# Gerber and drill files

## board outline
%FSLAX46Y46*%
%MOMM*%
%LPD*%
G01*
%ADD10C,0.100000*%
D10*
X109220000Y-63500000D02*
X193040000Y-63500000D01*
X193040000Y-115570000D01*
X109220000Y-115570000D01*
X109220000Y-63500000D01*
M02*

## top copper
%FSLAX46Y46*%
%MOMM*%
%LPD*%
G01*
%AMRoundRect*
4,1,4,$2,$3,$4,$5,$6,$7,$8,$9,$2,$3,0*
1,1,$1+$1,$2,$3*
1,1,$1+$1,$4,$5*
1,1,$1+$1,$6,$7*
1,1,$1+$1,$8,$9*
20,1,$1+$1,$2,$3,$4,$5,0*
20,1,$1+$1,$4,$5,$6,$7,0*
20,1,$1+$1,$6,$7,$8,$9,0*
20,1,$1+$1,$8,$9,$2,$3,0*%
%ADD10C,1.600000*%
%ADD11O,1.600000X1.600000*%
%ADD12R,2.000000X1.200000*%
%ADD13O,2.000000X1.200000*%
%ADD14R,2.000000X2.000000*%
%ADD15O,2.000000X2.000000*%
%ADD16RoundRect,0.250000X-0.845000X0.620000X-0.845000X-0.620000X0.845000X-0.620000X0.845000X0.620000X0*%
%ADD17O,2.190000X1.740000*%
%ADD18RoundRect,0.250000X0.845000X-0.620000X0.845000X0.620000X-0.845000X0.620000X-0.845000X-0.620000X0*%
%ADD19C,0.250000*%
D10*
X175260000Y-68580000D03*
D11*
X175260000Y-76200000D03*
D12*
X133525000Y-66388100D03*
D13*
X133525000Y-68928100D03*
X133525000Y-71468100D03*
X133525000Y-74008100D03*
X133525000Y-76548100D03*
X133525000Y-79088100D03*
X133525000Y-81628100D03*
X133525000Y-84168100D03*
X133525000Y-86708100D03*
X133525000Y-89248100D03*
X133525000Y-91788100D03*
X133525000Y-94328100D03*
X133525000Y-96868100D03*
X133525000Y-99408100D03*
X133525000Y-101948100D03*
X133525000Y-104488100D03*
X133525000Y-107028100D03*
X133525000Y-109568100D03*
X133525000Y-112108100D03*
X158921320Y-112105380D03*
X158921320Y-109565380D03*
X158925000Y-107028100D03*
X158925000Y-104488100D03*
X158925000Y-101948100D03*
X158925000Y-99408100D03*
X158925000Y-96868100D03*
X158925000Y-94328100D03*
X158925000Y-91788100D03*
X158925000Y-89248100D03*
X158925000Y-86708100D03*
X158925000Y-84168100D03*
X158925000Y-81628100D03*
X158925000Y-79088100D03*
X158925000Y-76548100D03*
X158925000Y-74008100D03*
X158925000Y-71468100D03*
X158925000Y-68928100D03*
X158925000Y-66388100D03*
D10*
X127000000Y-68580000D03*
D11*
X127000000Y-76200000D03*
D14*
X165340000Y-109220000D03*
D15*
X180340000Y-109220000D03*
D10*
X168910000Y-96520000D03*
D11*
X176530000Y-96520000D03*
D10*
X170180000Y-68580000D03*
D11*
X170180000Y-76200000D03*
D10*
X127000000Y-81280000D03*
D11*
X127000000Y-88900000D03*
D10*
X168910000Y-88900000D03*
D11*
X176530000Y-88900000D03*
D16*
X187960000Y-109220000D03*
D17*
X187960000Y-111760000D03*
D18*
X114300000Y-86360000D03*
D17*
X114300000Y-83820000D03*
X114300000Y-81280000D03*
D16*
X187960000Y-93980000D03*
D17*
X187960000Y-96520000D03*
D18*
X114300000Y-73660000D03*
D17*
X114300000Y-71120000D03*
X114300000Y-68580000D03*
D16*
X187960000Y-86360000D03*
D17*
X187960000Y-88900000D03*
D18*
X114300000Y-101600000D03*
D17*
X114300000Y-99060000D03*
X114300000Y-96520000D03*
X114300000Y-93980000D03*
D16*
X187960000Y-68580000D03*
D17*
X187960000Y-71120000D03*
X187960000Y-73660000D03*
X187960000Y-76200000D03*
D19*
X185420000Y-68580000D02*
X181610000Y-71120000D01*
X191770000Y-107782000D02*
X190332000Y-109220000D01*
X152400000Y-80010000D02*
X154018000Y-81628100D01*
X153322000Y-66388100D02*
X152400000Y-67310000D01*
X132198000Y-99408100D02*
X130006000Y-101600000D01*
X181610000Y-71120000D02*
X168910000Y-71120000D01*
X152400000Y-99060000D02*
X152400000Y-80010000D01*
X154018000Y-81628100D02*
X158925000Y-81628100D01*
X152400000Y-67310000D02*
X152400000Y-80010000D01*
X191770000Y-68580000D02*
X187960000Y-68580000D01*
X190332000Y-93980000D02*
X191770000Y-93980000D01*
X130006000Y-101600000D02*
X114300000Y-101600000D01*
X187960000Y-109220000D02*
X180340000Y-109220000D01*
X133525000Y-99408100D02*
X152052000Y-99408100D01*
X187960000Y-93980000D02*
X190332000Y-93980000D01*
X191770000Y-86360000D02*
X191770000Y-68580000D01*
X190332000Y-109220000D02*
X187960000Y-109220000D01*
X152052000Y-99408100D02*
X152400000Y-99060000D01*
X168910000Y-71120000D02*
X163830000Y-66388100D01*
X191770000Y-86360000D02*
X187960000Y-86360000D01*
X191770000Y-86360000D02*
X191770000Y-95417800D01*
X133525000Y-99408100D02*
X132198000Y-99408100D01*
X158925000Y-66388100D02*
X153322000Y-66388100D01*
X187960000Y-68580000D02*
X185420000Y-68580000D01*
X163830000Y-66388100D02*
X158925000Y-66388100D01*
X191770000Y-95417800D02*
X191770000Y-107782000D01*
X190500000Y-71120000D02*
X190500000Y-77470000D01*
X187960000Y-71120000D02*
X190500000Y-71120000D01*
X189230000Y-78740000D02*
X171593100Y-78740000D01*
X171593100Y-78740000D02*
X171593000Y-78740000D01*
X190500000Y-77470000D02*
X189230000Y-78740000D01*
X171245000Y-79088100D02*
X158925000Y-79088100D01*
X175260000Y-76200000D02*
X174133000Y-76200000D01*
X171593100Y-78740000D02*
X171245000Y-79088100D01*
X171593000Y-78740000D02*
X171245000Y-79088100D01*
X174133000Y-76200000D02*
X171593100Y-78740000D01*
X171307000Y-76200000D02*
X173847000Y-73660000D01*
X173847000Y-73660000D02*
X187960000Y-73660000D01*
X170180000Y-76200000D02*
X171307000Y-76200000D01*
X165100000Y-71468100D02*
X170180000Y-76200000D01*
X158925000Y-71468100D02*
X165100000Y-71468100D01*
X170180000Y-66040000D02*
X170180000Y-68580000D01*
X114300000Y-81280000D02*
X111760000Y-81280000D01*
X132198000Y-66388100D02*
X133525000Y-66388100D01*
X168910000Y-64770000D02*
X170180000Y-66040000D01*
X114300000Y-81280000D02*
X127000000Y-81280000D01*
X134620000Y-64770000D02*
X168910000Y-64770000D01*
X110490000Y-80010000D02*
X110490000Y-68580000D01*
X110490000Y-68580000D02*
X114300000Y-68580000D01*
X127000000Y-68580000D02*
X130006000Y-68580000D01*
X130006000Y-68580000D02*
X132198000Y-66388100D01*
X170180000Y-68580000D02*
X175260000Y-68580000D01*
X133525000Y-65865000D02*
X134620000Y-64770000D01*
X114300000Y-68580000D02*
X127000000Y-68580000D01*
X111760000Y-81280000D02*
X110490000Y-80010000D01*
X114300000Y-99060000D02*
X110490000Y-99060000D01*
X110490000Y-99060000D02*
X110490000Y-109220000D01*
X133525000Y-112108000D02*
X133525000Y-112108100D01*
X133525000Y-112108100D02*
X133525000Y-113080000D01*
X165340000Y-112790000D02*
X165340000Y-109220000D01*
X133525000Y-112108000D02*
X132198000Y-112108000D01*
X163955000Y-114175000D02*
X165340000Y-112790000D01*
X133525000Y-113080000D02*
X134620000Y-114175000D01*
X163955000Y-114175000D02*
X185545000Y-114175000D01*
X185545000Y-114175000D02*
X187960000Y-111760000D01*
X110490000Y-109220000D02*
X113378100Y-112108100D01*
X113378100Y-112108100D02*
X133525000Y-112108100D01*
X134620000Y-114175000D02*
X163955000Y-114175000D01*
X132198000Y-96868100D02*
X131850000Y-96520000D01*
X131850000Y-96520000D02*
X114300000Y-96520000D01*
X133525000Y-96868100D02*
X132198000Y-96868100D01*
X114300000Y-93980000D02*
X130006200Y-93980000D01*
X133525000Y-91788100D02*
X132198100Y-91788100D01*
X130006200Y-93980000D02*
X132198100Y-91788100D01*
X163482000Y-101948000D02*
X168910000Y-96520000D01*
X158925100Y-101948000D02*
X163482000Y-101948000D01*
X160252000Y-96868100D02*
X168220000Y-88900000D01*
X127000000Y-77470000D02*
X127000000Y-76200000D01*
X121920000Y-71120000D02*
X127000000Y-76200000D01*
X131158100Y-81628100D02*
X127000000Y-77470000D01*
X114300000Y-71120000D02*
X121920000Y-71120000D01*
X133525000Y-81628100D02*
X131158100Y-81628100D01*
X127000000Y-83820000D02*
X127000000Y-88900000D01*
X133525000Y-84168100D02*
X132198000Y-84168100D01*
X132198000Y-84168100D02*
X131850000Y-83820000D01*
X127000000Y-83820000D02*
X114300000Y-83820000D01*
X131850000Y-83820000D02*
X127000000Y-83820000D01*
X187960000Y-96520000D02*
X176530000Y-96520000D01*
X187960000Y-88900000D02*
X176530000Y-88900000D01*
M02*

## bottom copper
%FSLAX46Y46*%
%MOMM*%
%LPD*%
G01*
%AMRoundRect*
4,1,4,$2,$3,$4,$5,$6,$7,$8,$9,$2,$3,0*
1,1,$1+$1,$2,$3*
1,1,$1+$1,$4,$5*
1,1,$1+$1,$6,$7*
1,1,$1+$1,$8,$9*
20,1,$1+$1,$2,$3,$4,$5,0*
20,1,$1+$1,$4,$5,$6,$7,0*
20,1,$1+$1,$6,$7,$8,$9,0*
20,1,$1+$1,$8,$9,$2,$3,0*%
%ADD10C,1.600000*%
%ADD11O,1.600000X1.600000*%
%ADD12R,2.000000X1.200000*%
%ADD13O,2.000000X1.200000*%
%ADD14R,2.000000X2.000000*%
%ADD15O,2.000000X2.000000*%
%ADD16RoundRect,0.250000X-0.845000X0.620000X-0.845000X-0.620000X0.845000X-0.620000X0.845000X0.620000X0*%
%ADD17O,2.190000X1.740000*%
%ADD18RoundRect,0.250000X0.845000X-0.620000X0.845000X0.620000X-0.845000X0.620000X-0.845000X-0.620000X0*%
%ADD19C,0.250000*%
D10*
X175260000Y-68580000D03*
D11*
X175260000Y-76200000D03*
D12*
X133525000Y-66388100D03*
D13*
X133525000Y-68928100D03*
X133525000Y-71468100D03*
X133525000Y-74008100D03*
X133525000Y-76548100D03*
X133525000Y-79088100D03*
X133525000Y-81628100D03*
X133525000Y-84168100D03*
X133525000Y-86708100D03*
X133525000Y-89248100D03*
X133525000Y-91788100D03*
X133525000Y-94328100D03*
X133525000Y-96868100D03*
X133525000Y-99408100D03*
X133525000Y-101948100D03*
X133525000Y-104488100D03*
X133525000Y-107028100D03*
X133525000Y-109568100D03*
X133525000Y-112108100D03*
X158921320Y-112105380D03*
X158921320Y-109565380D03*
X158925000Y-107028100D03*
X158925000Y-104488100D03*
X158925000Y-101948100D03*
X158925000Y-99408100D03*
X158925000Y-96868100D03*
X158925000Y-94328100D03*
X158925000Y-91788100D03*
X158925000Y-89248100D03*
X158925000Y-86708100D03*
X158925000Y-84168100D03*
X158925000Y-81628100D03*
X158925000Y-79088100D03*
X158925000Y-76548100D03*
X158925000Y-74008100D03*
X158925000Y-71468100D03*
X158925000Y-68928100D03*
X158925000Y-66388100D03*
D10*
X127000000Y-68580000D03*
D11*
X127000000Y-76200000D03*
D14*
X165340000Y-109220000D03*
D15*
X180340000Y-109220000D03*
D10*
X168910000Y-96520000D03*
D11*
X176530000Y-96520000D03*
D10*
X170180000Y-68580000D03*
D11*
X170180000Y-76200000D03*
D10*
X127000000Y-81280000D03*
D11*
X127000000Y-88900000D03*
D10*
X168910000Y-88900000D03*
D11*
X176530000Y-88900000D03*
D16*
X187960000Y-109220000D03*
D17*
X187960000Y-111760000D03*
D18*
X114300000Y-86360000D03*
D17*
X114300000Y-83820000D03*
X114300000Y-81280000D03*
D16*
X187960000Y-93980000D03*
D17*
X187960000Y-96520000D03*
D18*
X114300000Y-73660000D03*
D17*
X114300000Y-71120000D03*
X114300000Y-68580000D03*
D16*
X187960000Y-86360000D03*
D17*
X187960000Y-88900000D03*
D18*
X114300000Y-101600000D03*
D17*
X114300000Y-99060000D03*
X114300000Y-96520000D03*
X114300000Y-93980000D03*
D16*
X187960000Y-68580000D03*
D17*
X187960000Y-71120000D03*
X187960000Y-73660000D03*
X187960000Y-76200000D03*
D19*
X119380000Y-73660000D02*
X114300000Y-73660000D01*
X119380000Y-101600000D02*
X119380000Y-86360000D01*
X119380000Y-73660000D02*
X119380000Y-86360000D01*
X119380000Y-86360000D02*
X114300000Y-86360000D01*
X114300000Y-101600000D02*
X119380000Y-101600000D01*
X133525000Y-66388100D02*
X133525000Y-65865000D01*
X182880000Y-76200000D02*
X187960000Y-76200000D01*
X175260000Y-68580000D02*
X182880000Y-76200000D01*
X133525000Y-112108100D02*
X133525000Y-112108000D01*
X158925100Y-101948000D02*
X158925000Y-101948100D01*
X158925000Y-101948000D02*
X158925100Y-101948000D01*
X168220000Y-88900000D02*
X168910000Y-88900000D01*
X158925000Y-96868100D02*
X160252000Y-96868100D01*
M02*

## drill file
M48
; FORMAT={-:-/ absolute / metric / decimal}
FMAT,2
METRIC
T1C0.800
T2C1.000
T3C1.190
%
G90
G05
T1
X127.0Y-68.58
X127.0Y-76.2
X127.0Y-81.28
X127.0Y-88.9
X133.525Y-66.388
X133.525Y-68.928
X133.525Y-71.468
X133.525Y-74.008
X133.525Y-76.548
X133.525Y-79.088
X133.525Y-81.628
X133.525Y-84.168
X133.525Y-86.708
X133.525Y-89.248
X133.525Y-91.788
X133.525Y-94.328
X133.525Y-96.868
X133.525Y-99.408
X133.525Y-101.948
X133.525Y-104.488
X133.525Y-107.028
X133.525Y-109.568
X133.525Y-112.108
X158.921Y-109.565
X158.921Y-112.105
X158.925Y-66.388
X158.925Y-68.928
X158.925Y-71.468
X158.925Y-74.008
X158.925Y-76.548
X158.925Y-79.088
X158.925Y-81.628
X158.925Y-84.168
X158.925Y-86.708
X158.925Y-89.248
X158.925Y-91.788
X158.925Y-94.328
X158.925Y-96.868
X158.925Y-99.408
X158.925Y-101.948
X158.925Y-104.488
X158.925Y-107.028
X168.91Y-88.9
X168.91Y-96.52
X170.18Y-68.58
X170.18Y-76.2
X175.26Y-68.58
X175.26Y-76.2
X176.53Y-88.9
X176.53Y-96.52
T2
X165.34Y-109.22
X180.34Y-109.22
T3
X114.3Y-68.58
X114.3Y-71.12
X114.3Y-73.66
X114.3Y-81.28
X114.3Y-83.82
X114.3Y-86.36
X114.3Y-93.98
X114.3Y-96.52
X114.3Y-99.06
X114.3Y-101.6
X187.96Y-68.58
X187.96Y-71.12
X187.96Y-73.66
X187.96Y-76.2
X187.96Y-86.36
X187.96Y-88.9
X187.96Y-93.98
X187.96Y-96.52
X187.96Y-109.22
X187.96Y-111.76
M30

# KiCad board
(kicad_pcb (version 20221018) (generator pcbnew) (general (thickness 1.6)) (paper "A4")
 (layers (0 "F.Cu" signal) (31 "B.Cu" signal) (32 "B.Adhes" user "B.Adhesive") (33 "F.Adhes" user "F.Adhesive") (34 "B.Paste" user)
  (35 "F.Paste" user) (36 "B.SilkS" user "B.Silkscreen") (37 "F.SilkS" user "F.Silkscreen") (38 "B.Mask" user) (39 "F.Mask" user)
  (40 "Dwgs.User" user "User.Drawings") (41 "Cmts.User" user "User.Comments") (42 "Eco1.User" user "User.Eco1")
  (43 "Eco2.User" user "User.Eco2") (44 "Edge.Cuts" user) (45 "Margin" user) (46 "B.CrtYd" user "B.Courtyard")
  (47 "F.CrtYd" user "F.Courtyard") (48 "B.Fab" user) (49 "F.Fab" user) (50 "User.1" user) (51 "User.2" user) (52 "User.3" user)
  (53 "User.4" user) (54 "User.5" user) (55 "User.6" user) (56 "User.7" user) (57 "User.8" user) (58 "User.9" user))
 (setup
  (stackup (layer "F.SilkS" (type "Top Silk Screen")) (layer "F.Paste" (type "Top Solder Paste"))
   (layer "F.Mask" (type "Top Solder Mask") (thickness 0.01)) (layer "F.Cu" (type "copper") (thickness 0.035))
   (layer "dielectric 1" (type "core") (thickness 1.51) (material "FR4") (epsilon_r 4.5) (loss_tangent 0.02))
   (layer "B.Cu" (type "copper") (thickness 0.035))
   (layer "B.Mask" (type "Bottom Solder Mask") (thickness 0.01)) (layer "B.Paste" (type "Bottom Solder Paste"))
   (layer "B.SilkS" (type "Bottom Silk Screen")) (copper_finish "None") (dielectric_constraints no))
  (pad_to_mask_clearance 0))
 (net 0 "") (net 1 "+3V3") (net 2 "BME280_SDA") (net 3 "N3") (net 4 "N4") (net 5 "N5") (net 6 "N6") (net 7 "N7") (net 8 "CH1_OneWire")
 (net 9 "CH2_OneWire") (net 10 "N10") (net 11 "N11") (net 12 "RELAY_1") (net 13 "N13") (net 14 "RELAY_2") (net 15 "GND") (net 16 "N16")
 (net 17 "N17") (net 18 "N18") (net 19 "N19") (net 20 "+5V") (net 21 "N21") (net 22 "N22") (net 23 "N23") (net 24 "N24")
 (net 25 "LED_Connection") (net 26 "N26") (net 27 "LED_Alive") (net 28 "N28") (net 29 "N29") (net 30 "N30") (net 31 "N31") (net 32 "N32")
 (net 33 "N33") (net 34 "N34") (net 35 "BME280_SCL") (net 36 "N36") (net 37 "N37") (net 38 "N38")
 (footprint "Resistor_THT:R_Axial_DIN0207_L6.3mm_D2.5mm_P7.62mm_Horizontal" (layer "F.Cu") (at 175.26 68.58 -90)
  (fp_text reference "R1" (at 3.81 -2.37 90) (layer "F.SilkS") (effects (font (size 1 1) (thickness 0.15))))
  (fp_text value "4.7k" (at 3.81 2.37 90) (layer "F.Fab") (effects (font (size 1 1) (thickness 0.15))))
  (pad "1" thru_hole circle (at 0 0 270) (size 1.6 1.6) (drill 0.8) (layers "*.Cu" "*.Mask") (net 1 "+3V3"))
  (pad "2" thru_hole oval (at 7.62 0 270) (size 1.6 1.6) (drill 0.8) (layers "*.Cu" "*.Mask") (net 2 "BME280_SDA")))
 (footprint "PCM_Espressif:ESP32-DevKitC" (layer "F.Cu") (at 133.525 66.3881)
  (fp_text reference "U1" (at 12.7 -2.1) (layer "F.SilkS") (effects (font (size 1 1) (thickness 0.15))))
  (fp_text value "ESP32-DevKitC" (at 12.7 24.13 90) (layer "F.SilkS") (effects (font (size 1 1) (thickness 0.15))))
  (pad "1" thru_hole rect (at 0 0 270) (size 1.2 2) (drill 0.8) (layers "*.Cu" "*.Mask") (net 1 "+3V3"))
  (pad "2" thru_hole oval (at 0 2.54 270) (size 1.2 2) (drill 0.8) (layers "*.Cu" "*.Mask") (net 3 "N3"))
  (pad "3" thru_hole oval (at 0 5.08 270) (size 1.2 2) (drill 0.8) (layers "*.Cu" "*.Mask") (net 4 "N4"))
  (pad "4" thru_hole oval (at 0 7.62 270) (size 1.2 2) (drill 0.8) (layers "*.Cu" "*.Mask") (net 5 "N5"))
  (pad "5" thru_hole oval (at 0 10.16 270) (size 1.2 2) (drill 0.8) (layers "*.Cu" "*.Mask") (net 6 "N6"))
  (pad "6" thru_hole oval (at 0 12.7 270) (size 1.2 2) (drill 0.8) (layers "*.Cu" "*.Mask") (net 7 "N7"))
  (pad "7" thru_hole oval (at 0 15.24 270) (size 1.2 2) (drill 0.8) (layers "*.Cu" "*.Mask") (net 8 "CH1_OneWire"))
  (pad "8" thru_hole oval (at 0 17.78 270) (size 1.2 2) (drill 0.8) (layers "*.Cu" "*.Mask") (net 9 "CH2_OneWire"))
  (pad "9" thru_hole oval (at 0 20.32 270) (size 1.2 2) (drill 0.8) (layers "*.Cu" "*.Mask") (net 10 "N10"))
  (pad "10" thru_hole oval (at 0 22.86 270) (size 1.2 2) (drill 0.8) (layers "*.Cu" "*.Mask") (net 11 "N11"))
  (pad "11" thru_hole oval (at 0 25.4 270) (size 1.2 2) (drill 0.8) (layers "*.Cu" "*.Mask") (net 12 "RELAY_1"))
  (pad "12" thru_hole oval (at 0 27.94 270) (size 1.2 2) (drill 0.8) (layers "*.Cu" "*.Mask") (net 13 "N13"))
  (pad "13" thru_hole oval (at 0 30.48 270) (size 1.2 2) (drill 0.8) (layers "*.Cu" "*.Mask") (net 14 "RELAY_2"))
  (pad "14" thru_hole oval (at 0 33.02 270) (size 1.2 2) (drill 0.8) (layers "*.Cu" "*.Mask") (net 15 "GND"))
  (pad "15" thru_hole oval (at 0 35.56 270) (size 1.2 2) (drill 0.8) (layers "*.Cu" "*.Mask") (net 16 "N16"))
  (pad "16" thru_hole oval (at 0 38.1 270) (size 1.2 2) (drill 0.8) (layers "*.Cu" "*.Mask") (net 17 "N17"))
  (pad "17" thru_hole oval (at 0 40.64 270) (size 1.2 2) (drill 0.8) (layers "*.Cu" "*.Mask") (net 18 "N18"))
  (pad "18" thru_hole oval (at 0 43.18 270) (size 1.2 2) (drill 0.8) (layers "*.Cu" "*.Mask") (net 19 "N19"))
  (pad "19" thru_hole oval (at 0 45.72 270) (size 1.2 2) (drill 0.8) (layers "*.Cu" "*.Mask") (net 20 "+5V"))
  (pad "20" thru_hole oval (at 25.39632 45.71728 270) (size 1.2 2) (drill 0.8) (layers "*.Cu" "*.Mask") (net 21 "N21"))
  (pad "21" thru_hole oval (at 25.39632 43.17728 270) (size 1.2 2) (drill 0.8) (layers "*.Cu" "*.Mask") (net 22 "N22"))
  (pad "22" thru_hole oval (at 25.4 40.64 270) (size 1.2 2) (drill 0.8) (layers "*.Cu" "*.Mask") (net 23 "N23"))
  (pad "23" thru_hole oval (at 25.4 38.1 270) (size 1.2 2) (drill 0.8) (layers "*.Cu" "*.Mask") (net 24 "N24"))
  (pad "24" thru_hole oval (at 25.4 35.56 270) (size 1.2 2) (drill 0.8) (layers "*.Cu" "*.Mask") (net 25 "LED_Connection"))
  (pad "25" thru_hole oval (at 25.4 33.02 270) (size 1.2 2) (drill 0.8) (layers "*.Cu" "*.Mask") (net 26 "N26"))
  (pad "26" thru_hole oval (at 25.4 30.48 270) (size 1.2 2) (drill 0.8) (layers "*.Cu" "*.Mask") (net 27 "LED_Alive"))
  (pad "27" thru_hole oval (at 25.4 27.94 270) (size 1.2 2) (drill 0.8) (layers "*.Cu" "*.Mask") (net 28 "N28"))
  (pad "28" thru_hole oval (at 25.4 25.4 270) (size 1.2 2) (drill 0.8) (layers "*.Cu" "*.Mask") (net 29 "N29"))
  (pad "29" thru_hole oval (at 25.4 22.86 270) (size 1.2 2) (drill 0.8) (layers "*.Cu" "*.Mask") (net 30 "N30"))
  (pad "30" thru_hole oval (at 25.4 20.32 270) (size 1.2 2) (drill 0.8) (layers "*.Cu" "*.Mask") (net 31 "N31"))
  (pad "31" thru_hole oval (at 25.4 17.78 270) (size 1.2 2) (drill 0.8) (layers "*.Cu" "*.Mask") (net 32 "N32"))
  (pad "32" thru_hole oval (at 25.4 15.24 270) (size 1.2 2) (drill 0.8) (layers "*.Cu" "*.Mask") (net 15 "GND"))
  (pad "33" thru_hole oval (at 25.4 12.7 270) (size 1.2 2) (drill 0.8) (layers "*.Cu" "*.Mask") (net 2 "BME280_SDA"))
  (pad "34" thru_hole oval (at 25.4 10.16 270) (size 1.2 2) (drill 0.8) (layers "*.Cu" "*.Mask") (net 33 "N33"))
  (pad "35" thru_hole oval (at 25.4 7.62 270) (size 1.2 2) (drill 0.8) (layers "*.Cu" "*.Mask") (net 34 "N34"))
  (pad "36" thru_hole oval (at 25.4 5.08 270) (size 1.2 2) (drill 0.8) (layers "*.Cu" "*.Mask") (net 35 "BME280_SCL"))
  (pad "37" thru_hole oval (at 25.4 2.54 270) (size 1.2 2) (drill 0.8) (layers "*.Cu" "*.Mask") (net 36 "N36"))
  (pad "38" thru_hole oval (at 25.4 0 270) (size 1.2 2) (drill 0.8) (layers "*.Cu" "*.Mask") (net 15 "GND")))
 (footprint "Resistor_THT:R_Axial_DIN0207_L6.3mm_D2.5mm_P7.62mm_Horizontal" (layer "F.Cu") (at 127 68.58 -90)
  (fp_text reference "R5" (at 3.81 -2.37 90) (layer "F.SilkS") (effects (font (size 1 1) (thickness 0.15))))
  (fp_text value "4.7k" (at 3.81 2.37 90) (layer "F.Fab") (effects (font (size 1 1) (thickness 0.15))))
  (pad "1" thru_hole circle (at 0 0 270) (size 1.6 1.6) (drill 0.8) (layers "*.Cu" "*.Mask") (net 1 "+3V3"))
  (pad "2" thru_hole oval (at 7.62 0 270) (size 1.6 1.6) (drill 0.8) (layers "*.Cu" "*.Mask") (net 8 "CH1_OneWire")))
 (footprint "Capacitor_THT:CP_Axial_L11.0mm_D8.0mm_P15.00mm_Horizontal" (layer "F.Cu") (at 165.34 109.22)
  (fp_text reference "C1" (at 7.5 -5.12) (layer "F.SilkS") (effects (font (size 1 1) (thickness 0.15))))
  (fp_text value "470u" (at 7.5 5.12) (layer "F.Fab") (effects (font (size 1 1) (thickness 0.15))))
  (pad "1" thru_hole rect (at 0 0) (size 2 2) (drill 1) (layers "*.Cu" "*.Mask") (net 20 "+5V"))
  (pad "2" thru_hole oval (at 15 0) (size 2 2) (drill 1) (layers "*.Cu" "*.Mask") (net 15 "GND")))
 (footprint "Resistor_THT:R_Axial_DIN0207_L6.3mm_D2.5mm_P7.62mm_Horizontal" (layer "F.Cu") (at 168.91 96.52)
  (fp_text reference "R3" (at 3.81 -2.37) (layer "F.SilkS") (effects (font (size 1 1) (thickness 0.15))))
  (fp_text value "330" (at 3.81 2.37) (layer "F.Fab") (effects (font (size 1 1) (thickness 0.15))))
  (pad "1" thru_hole circle (at 0 0) (size 1.6 1.6) (drill 0.8) (layers "*.Cu" "*.Mask") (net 25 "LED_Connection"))
  (pad "2" thru_hole oval (at 7.62 0) (size 1.6 1.6) (drill 0.8) (layers "*.Cu" "*.Mask") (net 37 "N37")))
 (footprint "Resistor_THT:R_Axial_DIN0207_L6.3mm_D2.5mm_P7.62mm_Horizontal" (layer "F.Cu") (at 170.18 68.58 -90)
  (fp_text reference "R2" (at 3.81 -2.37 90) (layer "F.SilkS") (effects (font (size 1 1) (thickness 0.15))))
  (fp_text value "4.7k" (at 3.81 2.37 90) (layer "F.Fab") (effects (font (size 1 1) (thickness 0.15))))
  (pad "1" thru_hole circle (at 0 0 270) (size 1.6 1.6) (drill 0.8) (layers "*.Cu" "*.Mask") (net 1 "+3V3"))
  (pad "2" thru_hole oval (at 7.62 0 270) (size 1.6 1.6) (drill 0.8) (layers "*.Cu" "*.Mask") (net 35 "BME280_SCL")))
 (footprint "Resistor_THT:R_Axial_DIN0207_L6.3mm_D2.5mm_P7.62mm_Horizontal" (layer "F.Cu") (at 127 81.28 -90)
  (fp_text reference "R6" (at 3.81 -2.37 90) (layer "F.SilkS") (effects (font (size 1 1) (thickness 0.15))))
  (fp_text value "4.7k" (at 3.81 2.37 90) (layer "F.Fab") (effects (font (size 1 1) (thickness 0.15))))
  (pad "1" thru_hole circle (at 0 0 270) (size 1.6 1.6) (drill 0.8) (layers "*.Cu" "*.Mask") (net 1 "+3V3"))
  (pad "2" thru_hole oval (at 7.62 0 270) (size 1.6 1.6) (drill 0.8) (layers "*.Cu" "*.Mask") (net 9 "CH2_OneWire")))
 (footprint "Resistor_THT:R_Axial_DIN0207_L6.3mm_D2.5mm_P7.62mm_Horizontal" (layer "F.Cu") (at 168.91 88.9)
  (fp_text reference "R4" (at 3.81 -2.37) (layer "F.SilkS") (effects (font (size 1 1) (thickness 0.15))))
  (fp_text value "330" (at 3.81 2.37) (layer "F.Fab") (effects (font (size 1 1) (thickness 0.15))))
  (pad "1" thru_hole circle (at 0 0) (size 1.6 1.6) (drill 0.8) (layers "*.Cu" "*.Mask") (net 27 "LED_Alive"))
  (pad "2" thru_hole oval (at 7.62 0) (size 1.6 1.6) (drill 0.8) (layers "*.Cu" "*.Mask") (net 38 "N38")))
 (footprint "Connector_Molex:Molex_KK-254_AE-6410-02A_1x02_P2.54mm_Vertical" (layer "F.Cu") (at 187.96 109.22 -90)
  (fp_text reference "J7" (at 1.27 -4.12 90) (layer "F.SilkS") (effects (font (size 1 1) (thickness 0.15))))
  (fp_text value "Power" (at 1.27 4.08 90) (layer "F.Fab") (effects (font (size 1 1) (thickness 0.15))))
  (pad "1" thru_hole roundrect (at 0 0 270) (size 1.74 2.19) (drill 1.19) (layers "*.Cu" "*.Mask") (roundrect_rratio 0.1436781609)
   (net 15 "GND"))
  (pad "2" thru_hole oval (at 2.54 0 270) (size 1.74 2.19) (drill 1.19) (layers "*.Cu" "*.Mask") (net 20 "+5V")))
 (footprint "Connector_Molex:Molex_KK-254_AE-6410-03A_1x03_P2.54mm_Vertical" (layer "F.Cu") (at 114.3 86.36 90)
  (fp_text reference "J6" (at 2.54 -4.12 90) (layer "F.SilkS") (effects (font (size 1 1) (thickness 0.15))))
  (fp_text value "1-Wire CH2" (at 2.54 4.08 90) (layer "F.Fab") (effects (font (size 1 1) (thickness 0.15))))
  (pad "1" thru_hole roundrect (at 0 0 90) (size 1.74 2.19) (drill 1.19) (layers "*.Cu" "*.Mask") (roundrect_rratio 0.1436781609)
   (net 15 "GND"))
  (pad "2" thru_hole oval (at 2.54 0 90) (size 1.74 2.19) (drill 1.19) (layers "*.Cu" "*.Mask") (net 9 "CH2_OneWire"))
  (pad "3" thru_hole oval (at 5.08 0 90) (size 1.74 2.19) (drill 1.19) (layers "*.Cu" "*.Mask") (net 1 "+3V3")))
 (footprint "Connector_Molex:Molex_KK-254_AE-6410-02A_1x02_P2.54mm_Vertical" (layer "F.Cu") (at 187.96 93.98 -90)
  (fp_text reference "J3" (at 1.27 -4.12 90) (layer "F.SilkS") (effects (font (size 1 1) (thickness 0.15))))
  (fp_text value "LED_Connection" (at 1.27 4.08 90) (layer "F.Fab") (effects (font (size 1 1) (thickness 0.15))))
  (pad "1" thru_hole roundrect (at 0 0 270) (size 1.74 2.19) (drill 1.19) (layers "*.Cu" "*.Mask") (roundrect_rratio 0.1436781609)
   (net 15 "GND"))
  (pad "2" thru_hole oval (at 2.54 0 270) (size 1.74 2.19) (drill 1.19) (layers "*.Cu" "*.Mask") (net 37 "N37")))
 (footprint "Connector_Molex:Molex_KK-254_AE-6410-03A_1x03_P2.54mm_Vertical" (layer "F.Cu") (at 114.3 73.66 90)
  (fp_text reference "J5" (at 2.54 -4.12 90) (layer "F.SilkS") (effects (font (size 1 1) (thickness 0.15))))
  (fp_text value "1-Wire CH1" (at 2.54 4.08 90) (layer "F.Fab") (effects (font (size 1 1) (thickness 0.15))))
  (pad "1" thru_hole roundrect (at 0 0 90) (size 1.74 2.19) (drill 1.19) (layers "*.Cu" "*.Mask") (roundrect_rratio 0.1436781609)
   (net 15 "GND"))
  (pad "2" thru_hole oval (at 2.54 0 90) (size 1.74 2.19) (drill 1.19) (layers "*.Cu" "*.Mask") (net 8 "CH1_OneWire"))
  (pad "3" thru_hole oval (at 5.08 0 90) (size 1.74 2.19) (drill 1.19) (layers "*.Cu" "*.Mask") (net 1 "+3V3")))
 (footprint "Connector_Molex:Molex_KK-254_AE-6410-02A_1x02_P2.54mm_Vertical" (layer "F.Cu") (at 187.96 86.36 -90)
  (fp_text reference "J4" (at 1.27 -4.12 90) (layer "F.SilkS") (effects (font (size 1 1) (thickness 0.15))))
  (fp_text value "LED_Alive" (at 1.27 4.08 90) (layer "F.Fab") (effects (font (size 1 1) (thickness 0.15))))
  (pad "1" thru_hole roundrect (at 0 0 270) (size 1.74 2.19) (drill 1.19) (layers "*.Cu" "*.Mask") (roundrect_rratio 0.1436781609)
   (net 15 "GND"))
  (pad "2" thru_hole oval (at 2.54 0 270) (size 1.74 2.19) (drill 1.19) (layers "*.Cu" "*.Mask") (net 38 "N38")))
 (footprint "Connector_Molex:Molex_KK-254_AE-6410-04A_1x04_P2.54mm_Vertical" (layer "F.Cu") (at 114.3 101.6 90)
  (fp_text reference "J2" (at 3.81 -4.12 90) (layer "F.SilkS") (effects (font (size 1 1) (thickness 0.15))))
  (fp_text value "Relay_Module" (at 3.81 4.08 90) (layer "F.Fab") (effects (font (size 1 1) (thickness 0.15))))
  (pad "1" thru_hole roundrect (at 0 0 90) (size 1.74 2.19) (drill 1.19) (layers "*.Cu" "*.Mask") (roundrect_rratio 0.1436781609)
   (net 15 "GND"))
  (pad "2" thru_hole oval (at 2.54 0 90) (size 1.74 2.19) (drill 1.19) (layers "*.Cu" "*.Mask") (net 20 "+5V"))
  (pad "3" thru_hole oval (at 5.08 0 90) (size 1.74 2.19) (drill 1.19) (layers "*.Cu" "*.Mask") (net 14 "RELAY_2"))
  (pad "4" thru_hole oval (at 7.62 0 90) (size 1.74 2.19) (drill 1.19) (layers "*.Cu" "*.Mask") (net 12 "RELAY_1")))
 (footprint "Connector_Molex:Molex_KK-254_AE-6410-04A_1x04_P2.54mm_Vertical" (layer "F.Cu") (at 187.96 68.58 -90)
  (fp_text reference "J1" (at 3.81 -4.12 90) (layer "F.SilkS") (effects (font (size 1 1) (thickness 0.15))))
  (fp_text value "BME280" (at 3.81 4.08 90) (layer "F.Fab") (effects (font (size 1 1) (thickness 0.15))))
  (pad "1" thru_hole roundrect (at 0 0 270) (size 1.74 2.19) (drill 1.19) (layers "*.Cu" "*.Mask") (roundrect_rratio 0.1436781609)
   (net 15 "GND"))
  (pad "2" thru_hole oval (at 2.54 0 270) (size 1.74 2.19) (drill 1.19) (layers "*.Cu" "*.Mask") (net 2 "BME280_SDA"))
  (pad "3" thru_hole oval (at 5.08 0 270) (size 1.74 2.19) (drill 1.19) (layers "*.Cu" "*.Mask") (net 35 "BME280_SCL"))
  (pad "4" thru_hole oval (at 7.62 0 270) (size 1.74 2.19) (drill 1.19) (layers "*.Cu" "*.Mask") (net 1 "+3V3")))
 (gr_rect (start 109.22 63.5) (end 193.04 115.57) (stroke (width 0.1) (type default)) (fill none) (layer "Edge.Cuts"))
 (segment (start 185.42 68.58) (end 181.61 71.12) (width 0.25) (layer "F.Cu") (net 15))
 (segment (start 191.77 107.782) (end 190.332 109.22) (width 0.25) (layer "F.Cu") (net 15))
 (segment (start 152.4 80.01) (end 154.018 81.6281) (width 0.25) (layer "F.Cu") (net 15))
 (segment (start 153.322 66.3881) (end 152.4 67.31) (width 0.25) (layer "F.Cu") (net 15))
 (segment (start 132.198 99.4081) (end 130.006 101.6) (width 0.25) (layer "F.Cu") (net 15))
 (segment (start 181.61 71.12) (end 168.91 71.12) (width 0.25) (layer "F.Cu") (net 15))
 (segment (start 152.4 99.06) (end 152.4 80.01) (width 0.25) (layer "F.Cu") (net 15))
 (segment (start 154.018 81.6281) (end 158.925 81.6281) (width 0.25) (layer "F.Cu") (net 15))
 (segment (start 152.4 67.31) (end 152.4 80.01) (width 0.25) (layer "F.Cu") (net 15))
 (segment (start 191.77 68.58) (end 187.96 68.58) (width 0.25) (layer "F.Cu") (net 15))
 (segment (start 190.332 93.98) (end 191.77 93.98) (width 0.25) (layer "F.Cu") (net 15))
 (segment (start 130.006 101.6) (end 114.3 101.6) (width 0.25) (layer "F.Cu") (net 15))
 (segment (start 187.96 109.22) (end 180.34 109.22) (width 0.25) (layer "F.Cu") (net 15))
 (segment (start 133.525 99.4081) (end 152.052 99.4081) (width 0.25) (layer "F.Cu") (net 15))
 (segment (start 187.96 93.98) (end 190.332 93.98) (width 0.25) (layer "F.Cu") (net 15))
 (segment (start 191.77 86.36) (end 191.77 68.58) (width 0.25) (layer "F.Cu") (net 15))
 (segment (start 190.332 109.22) (end 187.96 109.22) (width 0.25) (layer "F.Cu") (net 15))
 (segment (start 152.052 99.4081) (end 152.4 99.06) (width 0.25) (layer "F.Cu") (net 15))
 (segment (start 168.91 71.12) (end 163.83 66.3881) (width 0.25) (layer "F.Cu") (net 15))
 (segment (start 191.77 86.36) (end 187.96 86.36) (width 0.25) (layer "F.Cu") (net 15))
 (segment (start 191.77 86.36) (end 191.77 95.4178) (width 0.25) (layer "F.Cu") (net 15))
 (segment (start 133.525 99.4081) (end 132.198 99.4081) (width 0.25) (layer "F.Cu") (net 15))
 (segment (start 158.925 66.3881) (end 153.322 66.3881) (width 0.25) (layer "F.Cu") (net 15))
 (segment (start 187.96 68.58) (end 185.42 68.58) (width 0.25) (layer "F.Cu") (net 15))
 (segment (start 163.83 66.3881) (end 158.925 66.3881) (width 0.25) (layer "F.Cu") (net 15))
 (segment (start 191.77 95.4178) (end 191.77 107.782) (width 0.25) (layer "F.Cu") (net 15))
 (segment (start 119.38 73.66) (end 114.3 73.66) (width 0.25) (layer "B.Cu") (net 15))
 (segment (start 119.38 101.6) (end 119.38 86.36) (width 0.25) (layer "B.Cu") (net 15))
 (segment (start 119.38 73.66) (end 119.38 86.36) (width 0.25) (layer "B.Cu") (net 15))
 (segment (start 119.38 86.36) (end 114.3 86.36) (width 0.25) (layer "B.Cu") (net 15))
 (segment (start 114.3 101.6) (end 119.38 101.6) (width 0.25) (layer "B.Cu") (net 15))
 (segment (start 190.5 71.12) (end 190.5 77.47) (width 0.25) (layer "F.Cu") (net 2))
 (segment (start 187.96 71.12) (end 190.5 71.12) (width 0.25) (layer "F.Cu") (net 2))
 (segment (start 189.23 78.74) (end 171.5931 78.74) (width 0.25) (layer "F.Cu") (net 2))
 (segment (start 171.5931 78.74) (end 171.593 78.74) (width 0.25) (layer "F.Cu") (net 2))
 (segment (start 190.5 77.47) (end 189.23 78.74) (width 0.25) (layer "F.Cu") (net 2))
 (segment (start 171.245 79.0881) (end 158.925 79.0881) (width 0.25) (layer "F.Cu") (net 2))
 (segment (start 175.26 76.2) (end 174.133 76.2) (width 0.25) (layer "F.Cu") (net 2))
 (segment (start 171.5931 78.74) (end 171.245 79.0881) (width 0.25) (layer "F.Cu") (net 2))
 (segment (start 171.593 78.74) (end 171.245 79.0881) (width 0.25) (layer "F.Cu") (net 2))
 (segment (start 174.133 76.2) (end 171.5931 78.74) (width 0.25) (layer "F.Cu") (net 2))
 (segment (start 171.307 76.2) (end 173.847 73.66) (width 0.25) (layer "F.Cu") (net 35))
 (segment (start 173.847 73.66) (end 187.96 73.66) (width 0.25) (layer "F.Cu") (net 35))
 (segment (start 170.18 76.2) (end 171.307 76.2) (width 0.25) (layer "F.Cu") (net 35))
 (segment (start 165.1 71.4681) (end 170.18 76.2) (width 0.25) (layer "F.Cu") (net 35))
 (segment (start 158.925 71.4681) (end 165.1 71.4681) (width 0.25) (layer "F.Cu") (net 35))
 (segment (start 170.18 66.04) (end 170.18 68.58) (width 0.25) (layer "F.Cu") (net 1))
 (segment (start 114.3 81.28) (end 111.76 81.28) (width 0.25) (layer "F.Cu") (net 1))
 (segment (start 132.198 66.3881) (end 133.525 66.3881) (width 0.25) (layer "F.Cu") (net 1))
 (segment (start 168.91 64.77) (end 170.18 66.04) (width 0.25) (layer "F.Cu") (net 1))
 (segment (start 114.3 81.28) (end 127 81.28) (width 0.25) (layer "F.Cu") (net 1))
 (segment (start 134.62 64.77) (end 168.91 64.77) (width 0.25) (layer "F.Cu") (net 1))
 (segment (start 110.49 80.01) (end 110.49 68.58) (width 0.25) (layer "F.Cu") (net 1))
 (segment (start 110.49 68.58) (end 114.3 68.58) (width 0.25) (layer "F.Cu") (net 1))
 (segment (start 127 68.58) (end 130.006 68.58) (width 0.25) (layer "F.Cu") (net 1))
 (segment (start 130.006 68.58) (end 132.198 66.3881) (width 0.25) (layer "F.Cu") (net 1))
 (segment (start 170.18 68.58) (end 175.26 68.58) (width 0.25) (layer "F.Cu") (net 1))
 (segment (start 133.525 65.865) (end 134.62 64.77) (width 0.25) (layer "F.Cu") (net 1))
 (segment (start 114.3 68.58) (end 127 68.58) (width 0.25) (layer "F.Cu") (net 1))
 (segment (start 111.76 81.28) (end 110.49 80.01) (width 0.25) (layer "F.Cu") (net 1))
 (segment (start 133.525 66.3881) (end 133.525 65.865) (width 0.25) (layer "B.Cu") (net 1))
 (segment (start 182.88 76.2) (end 187.96 76.2) (width 0.25) (layer "B.Cu") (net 1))
 (segment (start 175.26 68.58) (end 182.88 76.2) (width 0.25) (layer "B.Cu") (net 1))
 (segment (start 114.3 99.06) (end 110.49 99.06) (width 0.25) (layer "F.Cu") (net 20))
 (segment (start 110.49 99.06) (end 110.49 109.22) (width 0.25) (layer "F.Cu") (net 20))
 (segment (start 133.525 112.108) (end 133.525 112.1081) (width 0.25) (layer "F.Cu") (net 20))
 (segment (start 133.525 112.1081) (end 133.525 113.08) (width 0.25) (layer "F.Cu") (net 20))
 (segment (start 165.34 112.79) (end 165.34 109.22) (width 0.25) (layer "F.Cu") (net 20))
 (segment (start 133.525 112.108) (end 132.198 112.108) (width 0.25) (layer "F.Cu") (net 20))
 (segment (start 163.955 114.175) (end 165.34 112.79) (width 0.25) (layer "F.Cu") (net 20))
 (segment (start 133.525 113.08) (end 134.62 114.175) (width 0.25) (layer "F.Cu") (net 20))
 (segment (start 163.955 114.175) (end 185.545 114.175) (width 0.25) (layer "F.Cu") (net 20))
 (segment (start 185.545 114.175) (end 187.96 111.76) (width 0.25) (layer "F.Cu") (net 20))
 (segment (start 110.49 109.22) (end 113.3781 112.1081) (width 0.25) (layer "F.Cu") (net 20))
 (segment (start 113.3781 112.1081) (end 133.525 112.1081) (width 0.25) (layer "F.Cu") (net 20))
 (segment (start 134.62 114.175) (end 163.955 114.175) (width 0.25) (layer "F.Cu") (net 20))
 (segment (start 133.525 112.1081) (end 133.525 112.108) (width 0.25) (layer "B.Cu") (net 20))
 (segment (start 132.198 96.8681) (end 131.85 96.52) (width 0.25) (layer "F.Cu") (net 14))
 (segment (start 131.85 96.52) (end 114.3 96.52) (width 0.25) (layer "F.Cu") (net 14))
 (segment (start 133.525 96.8681) (end 132.198 96.8681) (width 0.25) (layer "F.Cu") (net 14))
 (segment (start 114.3 93.98) (end 130.0062 93.98) (width 0.25) (layer "F.Cu") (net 12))
 (segment (start 133.525 91.7881) (end 132.1981 91.7881) (width 0.25) (layer "F.Cu") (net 12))
 (segment (start 130.0062 93.98) (end 132.1981 91.7881) (width 0.25) (layer "F.Cu") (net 12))
 (segment (start 163.482 101.948) (end 168.91 96.52) (width 0.25) (layer "F.Cu") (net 25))
 (segment (start 158.9251 101.948) (end 163.482 101.948) (width 0.25) (layer "F.Cu") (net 25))
 (segment (start 158.9251 101.948) (end 158.925 101.9481) (width 0.25) (layer "B.Cu") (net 25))
 (segment (start 158.925 101.948) (end 158.9251 101.948) (width 0.25) (layer "B.Cu") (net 25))
 (segment (start 160.252 96.8681) (end 168.22 88.9) (width 0.25) (layer "F.Cu") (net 27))
 (segment (start 168.22 88.9) (end 168.91 88.9) (width 0.25) (layer "B.Cu") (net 27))
 (segment (start 158.925 96.8681) (end 160.252 96.8681) (width 0.25) (layer "B.Cu") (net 27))
 (segment (start 127 77.47) (end 127 76.2) (width 0.25) (layer "F.Cu") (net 8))
 (segment (start 121.92 71.12) (end 127 76.2) (width 0.25) (layer "F.Cu") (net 8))
 (segment (start 131.1581 81.6281) (end 127 77.47) (width 0.25) (layer "F.Cu") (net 8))
 (segment (start 114.3 71.12) (end 121.92 71.12) (width 0.25) (layer "F.Cu") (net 8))
 (segment (start 133.525 81.6281) (end 131.1581 81.6281) (width 0.25) (layer "F.Cu") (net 8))
 (segment (start 127 83.82) (end 127 88.9) (width 0.25) (layer "F.Cu") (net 9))
 (segment (start 133.525 84.1681) (end 132.198 84.1681) (width 0.25) (layer "F.Cu") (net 9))
 (segment (start 132.198 84.1681) (end 131.85 83.82) (width 0.25) (layer "F.Cu") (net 9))
 (segment (start 127 83.82) (end 114.3 83.82) (width 0.25) (layer "F.Cu") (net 9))
 (segment (start 131.85 83.82) (end 127 83.82) (width 0.25) (layer "F.Cu") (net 9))
 (segment (start 187.96 96.52) (end 176.53 96.52) (width 0.25) (layer "F.Cu") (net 37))
 (segment (start 187.96 88.9) (end 176.53 88.9) (width 0.25) (layer "F.Cu") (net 38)))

